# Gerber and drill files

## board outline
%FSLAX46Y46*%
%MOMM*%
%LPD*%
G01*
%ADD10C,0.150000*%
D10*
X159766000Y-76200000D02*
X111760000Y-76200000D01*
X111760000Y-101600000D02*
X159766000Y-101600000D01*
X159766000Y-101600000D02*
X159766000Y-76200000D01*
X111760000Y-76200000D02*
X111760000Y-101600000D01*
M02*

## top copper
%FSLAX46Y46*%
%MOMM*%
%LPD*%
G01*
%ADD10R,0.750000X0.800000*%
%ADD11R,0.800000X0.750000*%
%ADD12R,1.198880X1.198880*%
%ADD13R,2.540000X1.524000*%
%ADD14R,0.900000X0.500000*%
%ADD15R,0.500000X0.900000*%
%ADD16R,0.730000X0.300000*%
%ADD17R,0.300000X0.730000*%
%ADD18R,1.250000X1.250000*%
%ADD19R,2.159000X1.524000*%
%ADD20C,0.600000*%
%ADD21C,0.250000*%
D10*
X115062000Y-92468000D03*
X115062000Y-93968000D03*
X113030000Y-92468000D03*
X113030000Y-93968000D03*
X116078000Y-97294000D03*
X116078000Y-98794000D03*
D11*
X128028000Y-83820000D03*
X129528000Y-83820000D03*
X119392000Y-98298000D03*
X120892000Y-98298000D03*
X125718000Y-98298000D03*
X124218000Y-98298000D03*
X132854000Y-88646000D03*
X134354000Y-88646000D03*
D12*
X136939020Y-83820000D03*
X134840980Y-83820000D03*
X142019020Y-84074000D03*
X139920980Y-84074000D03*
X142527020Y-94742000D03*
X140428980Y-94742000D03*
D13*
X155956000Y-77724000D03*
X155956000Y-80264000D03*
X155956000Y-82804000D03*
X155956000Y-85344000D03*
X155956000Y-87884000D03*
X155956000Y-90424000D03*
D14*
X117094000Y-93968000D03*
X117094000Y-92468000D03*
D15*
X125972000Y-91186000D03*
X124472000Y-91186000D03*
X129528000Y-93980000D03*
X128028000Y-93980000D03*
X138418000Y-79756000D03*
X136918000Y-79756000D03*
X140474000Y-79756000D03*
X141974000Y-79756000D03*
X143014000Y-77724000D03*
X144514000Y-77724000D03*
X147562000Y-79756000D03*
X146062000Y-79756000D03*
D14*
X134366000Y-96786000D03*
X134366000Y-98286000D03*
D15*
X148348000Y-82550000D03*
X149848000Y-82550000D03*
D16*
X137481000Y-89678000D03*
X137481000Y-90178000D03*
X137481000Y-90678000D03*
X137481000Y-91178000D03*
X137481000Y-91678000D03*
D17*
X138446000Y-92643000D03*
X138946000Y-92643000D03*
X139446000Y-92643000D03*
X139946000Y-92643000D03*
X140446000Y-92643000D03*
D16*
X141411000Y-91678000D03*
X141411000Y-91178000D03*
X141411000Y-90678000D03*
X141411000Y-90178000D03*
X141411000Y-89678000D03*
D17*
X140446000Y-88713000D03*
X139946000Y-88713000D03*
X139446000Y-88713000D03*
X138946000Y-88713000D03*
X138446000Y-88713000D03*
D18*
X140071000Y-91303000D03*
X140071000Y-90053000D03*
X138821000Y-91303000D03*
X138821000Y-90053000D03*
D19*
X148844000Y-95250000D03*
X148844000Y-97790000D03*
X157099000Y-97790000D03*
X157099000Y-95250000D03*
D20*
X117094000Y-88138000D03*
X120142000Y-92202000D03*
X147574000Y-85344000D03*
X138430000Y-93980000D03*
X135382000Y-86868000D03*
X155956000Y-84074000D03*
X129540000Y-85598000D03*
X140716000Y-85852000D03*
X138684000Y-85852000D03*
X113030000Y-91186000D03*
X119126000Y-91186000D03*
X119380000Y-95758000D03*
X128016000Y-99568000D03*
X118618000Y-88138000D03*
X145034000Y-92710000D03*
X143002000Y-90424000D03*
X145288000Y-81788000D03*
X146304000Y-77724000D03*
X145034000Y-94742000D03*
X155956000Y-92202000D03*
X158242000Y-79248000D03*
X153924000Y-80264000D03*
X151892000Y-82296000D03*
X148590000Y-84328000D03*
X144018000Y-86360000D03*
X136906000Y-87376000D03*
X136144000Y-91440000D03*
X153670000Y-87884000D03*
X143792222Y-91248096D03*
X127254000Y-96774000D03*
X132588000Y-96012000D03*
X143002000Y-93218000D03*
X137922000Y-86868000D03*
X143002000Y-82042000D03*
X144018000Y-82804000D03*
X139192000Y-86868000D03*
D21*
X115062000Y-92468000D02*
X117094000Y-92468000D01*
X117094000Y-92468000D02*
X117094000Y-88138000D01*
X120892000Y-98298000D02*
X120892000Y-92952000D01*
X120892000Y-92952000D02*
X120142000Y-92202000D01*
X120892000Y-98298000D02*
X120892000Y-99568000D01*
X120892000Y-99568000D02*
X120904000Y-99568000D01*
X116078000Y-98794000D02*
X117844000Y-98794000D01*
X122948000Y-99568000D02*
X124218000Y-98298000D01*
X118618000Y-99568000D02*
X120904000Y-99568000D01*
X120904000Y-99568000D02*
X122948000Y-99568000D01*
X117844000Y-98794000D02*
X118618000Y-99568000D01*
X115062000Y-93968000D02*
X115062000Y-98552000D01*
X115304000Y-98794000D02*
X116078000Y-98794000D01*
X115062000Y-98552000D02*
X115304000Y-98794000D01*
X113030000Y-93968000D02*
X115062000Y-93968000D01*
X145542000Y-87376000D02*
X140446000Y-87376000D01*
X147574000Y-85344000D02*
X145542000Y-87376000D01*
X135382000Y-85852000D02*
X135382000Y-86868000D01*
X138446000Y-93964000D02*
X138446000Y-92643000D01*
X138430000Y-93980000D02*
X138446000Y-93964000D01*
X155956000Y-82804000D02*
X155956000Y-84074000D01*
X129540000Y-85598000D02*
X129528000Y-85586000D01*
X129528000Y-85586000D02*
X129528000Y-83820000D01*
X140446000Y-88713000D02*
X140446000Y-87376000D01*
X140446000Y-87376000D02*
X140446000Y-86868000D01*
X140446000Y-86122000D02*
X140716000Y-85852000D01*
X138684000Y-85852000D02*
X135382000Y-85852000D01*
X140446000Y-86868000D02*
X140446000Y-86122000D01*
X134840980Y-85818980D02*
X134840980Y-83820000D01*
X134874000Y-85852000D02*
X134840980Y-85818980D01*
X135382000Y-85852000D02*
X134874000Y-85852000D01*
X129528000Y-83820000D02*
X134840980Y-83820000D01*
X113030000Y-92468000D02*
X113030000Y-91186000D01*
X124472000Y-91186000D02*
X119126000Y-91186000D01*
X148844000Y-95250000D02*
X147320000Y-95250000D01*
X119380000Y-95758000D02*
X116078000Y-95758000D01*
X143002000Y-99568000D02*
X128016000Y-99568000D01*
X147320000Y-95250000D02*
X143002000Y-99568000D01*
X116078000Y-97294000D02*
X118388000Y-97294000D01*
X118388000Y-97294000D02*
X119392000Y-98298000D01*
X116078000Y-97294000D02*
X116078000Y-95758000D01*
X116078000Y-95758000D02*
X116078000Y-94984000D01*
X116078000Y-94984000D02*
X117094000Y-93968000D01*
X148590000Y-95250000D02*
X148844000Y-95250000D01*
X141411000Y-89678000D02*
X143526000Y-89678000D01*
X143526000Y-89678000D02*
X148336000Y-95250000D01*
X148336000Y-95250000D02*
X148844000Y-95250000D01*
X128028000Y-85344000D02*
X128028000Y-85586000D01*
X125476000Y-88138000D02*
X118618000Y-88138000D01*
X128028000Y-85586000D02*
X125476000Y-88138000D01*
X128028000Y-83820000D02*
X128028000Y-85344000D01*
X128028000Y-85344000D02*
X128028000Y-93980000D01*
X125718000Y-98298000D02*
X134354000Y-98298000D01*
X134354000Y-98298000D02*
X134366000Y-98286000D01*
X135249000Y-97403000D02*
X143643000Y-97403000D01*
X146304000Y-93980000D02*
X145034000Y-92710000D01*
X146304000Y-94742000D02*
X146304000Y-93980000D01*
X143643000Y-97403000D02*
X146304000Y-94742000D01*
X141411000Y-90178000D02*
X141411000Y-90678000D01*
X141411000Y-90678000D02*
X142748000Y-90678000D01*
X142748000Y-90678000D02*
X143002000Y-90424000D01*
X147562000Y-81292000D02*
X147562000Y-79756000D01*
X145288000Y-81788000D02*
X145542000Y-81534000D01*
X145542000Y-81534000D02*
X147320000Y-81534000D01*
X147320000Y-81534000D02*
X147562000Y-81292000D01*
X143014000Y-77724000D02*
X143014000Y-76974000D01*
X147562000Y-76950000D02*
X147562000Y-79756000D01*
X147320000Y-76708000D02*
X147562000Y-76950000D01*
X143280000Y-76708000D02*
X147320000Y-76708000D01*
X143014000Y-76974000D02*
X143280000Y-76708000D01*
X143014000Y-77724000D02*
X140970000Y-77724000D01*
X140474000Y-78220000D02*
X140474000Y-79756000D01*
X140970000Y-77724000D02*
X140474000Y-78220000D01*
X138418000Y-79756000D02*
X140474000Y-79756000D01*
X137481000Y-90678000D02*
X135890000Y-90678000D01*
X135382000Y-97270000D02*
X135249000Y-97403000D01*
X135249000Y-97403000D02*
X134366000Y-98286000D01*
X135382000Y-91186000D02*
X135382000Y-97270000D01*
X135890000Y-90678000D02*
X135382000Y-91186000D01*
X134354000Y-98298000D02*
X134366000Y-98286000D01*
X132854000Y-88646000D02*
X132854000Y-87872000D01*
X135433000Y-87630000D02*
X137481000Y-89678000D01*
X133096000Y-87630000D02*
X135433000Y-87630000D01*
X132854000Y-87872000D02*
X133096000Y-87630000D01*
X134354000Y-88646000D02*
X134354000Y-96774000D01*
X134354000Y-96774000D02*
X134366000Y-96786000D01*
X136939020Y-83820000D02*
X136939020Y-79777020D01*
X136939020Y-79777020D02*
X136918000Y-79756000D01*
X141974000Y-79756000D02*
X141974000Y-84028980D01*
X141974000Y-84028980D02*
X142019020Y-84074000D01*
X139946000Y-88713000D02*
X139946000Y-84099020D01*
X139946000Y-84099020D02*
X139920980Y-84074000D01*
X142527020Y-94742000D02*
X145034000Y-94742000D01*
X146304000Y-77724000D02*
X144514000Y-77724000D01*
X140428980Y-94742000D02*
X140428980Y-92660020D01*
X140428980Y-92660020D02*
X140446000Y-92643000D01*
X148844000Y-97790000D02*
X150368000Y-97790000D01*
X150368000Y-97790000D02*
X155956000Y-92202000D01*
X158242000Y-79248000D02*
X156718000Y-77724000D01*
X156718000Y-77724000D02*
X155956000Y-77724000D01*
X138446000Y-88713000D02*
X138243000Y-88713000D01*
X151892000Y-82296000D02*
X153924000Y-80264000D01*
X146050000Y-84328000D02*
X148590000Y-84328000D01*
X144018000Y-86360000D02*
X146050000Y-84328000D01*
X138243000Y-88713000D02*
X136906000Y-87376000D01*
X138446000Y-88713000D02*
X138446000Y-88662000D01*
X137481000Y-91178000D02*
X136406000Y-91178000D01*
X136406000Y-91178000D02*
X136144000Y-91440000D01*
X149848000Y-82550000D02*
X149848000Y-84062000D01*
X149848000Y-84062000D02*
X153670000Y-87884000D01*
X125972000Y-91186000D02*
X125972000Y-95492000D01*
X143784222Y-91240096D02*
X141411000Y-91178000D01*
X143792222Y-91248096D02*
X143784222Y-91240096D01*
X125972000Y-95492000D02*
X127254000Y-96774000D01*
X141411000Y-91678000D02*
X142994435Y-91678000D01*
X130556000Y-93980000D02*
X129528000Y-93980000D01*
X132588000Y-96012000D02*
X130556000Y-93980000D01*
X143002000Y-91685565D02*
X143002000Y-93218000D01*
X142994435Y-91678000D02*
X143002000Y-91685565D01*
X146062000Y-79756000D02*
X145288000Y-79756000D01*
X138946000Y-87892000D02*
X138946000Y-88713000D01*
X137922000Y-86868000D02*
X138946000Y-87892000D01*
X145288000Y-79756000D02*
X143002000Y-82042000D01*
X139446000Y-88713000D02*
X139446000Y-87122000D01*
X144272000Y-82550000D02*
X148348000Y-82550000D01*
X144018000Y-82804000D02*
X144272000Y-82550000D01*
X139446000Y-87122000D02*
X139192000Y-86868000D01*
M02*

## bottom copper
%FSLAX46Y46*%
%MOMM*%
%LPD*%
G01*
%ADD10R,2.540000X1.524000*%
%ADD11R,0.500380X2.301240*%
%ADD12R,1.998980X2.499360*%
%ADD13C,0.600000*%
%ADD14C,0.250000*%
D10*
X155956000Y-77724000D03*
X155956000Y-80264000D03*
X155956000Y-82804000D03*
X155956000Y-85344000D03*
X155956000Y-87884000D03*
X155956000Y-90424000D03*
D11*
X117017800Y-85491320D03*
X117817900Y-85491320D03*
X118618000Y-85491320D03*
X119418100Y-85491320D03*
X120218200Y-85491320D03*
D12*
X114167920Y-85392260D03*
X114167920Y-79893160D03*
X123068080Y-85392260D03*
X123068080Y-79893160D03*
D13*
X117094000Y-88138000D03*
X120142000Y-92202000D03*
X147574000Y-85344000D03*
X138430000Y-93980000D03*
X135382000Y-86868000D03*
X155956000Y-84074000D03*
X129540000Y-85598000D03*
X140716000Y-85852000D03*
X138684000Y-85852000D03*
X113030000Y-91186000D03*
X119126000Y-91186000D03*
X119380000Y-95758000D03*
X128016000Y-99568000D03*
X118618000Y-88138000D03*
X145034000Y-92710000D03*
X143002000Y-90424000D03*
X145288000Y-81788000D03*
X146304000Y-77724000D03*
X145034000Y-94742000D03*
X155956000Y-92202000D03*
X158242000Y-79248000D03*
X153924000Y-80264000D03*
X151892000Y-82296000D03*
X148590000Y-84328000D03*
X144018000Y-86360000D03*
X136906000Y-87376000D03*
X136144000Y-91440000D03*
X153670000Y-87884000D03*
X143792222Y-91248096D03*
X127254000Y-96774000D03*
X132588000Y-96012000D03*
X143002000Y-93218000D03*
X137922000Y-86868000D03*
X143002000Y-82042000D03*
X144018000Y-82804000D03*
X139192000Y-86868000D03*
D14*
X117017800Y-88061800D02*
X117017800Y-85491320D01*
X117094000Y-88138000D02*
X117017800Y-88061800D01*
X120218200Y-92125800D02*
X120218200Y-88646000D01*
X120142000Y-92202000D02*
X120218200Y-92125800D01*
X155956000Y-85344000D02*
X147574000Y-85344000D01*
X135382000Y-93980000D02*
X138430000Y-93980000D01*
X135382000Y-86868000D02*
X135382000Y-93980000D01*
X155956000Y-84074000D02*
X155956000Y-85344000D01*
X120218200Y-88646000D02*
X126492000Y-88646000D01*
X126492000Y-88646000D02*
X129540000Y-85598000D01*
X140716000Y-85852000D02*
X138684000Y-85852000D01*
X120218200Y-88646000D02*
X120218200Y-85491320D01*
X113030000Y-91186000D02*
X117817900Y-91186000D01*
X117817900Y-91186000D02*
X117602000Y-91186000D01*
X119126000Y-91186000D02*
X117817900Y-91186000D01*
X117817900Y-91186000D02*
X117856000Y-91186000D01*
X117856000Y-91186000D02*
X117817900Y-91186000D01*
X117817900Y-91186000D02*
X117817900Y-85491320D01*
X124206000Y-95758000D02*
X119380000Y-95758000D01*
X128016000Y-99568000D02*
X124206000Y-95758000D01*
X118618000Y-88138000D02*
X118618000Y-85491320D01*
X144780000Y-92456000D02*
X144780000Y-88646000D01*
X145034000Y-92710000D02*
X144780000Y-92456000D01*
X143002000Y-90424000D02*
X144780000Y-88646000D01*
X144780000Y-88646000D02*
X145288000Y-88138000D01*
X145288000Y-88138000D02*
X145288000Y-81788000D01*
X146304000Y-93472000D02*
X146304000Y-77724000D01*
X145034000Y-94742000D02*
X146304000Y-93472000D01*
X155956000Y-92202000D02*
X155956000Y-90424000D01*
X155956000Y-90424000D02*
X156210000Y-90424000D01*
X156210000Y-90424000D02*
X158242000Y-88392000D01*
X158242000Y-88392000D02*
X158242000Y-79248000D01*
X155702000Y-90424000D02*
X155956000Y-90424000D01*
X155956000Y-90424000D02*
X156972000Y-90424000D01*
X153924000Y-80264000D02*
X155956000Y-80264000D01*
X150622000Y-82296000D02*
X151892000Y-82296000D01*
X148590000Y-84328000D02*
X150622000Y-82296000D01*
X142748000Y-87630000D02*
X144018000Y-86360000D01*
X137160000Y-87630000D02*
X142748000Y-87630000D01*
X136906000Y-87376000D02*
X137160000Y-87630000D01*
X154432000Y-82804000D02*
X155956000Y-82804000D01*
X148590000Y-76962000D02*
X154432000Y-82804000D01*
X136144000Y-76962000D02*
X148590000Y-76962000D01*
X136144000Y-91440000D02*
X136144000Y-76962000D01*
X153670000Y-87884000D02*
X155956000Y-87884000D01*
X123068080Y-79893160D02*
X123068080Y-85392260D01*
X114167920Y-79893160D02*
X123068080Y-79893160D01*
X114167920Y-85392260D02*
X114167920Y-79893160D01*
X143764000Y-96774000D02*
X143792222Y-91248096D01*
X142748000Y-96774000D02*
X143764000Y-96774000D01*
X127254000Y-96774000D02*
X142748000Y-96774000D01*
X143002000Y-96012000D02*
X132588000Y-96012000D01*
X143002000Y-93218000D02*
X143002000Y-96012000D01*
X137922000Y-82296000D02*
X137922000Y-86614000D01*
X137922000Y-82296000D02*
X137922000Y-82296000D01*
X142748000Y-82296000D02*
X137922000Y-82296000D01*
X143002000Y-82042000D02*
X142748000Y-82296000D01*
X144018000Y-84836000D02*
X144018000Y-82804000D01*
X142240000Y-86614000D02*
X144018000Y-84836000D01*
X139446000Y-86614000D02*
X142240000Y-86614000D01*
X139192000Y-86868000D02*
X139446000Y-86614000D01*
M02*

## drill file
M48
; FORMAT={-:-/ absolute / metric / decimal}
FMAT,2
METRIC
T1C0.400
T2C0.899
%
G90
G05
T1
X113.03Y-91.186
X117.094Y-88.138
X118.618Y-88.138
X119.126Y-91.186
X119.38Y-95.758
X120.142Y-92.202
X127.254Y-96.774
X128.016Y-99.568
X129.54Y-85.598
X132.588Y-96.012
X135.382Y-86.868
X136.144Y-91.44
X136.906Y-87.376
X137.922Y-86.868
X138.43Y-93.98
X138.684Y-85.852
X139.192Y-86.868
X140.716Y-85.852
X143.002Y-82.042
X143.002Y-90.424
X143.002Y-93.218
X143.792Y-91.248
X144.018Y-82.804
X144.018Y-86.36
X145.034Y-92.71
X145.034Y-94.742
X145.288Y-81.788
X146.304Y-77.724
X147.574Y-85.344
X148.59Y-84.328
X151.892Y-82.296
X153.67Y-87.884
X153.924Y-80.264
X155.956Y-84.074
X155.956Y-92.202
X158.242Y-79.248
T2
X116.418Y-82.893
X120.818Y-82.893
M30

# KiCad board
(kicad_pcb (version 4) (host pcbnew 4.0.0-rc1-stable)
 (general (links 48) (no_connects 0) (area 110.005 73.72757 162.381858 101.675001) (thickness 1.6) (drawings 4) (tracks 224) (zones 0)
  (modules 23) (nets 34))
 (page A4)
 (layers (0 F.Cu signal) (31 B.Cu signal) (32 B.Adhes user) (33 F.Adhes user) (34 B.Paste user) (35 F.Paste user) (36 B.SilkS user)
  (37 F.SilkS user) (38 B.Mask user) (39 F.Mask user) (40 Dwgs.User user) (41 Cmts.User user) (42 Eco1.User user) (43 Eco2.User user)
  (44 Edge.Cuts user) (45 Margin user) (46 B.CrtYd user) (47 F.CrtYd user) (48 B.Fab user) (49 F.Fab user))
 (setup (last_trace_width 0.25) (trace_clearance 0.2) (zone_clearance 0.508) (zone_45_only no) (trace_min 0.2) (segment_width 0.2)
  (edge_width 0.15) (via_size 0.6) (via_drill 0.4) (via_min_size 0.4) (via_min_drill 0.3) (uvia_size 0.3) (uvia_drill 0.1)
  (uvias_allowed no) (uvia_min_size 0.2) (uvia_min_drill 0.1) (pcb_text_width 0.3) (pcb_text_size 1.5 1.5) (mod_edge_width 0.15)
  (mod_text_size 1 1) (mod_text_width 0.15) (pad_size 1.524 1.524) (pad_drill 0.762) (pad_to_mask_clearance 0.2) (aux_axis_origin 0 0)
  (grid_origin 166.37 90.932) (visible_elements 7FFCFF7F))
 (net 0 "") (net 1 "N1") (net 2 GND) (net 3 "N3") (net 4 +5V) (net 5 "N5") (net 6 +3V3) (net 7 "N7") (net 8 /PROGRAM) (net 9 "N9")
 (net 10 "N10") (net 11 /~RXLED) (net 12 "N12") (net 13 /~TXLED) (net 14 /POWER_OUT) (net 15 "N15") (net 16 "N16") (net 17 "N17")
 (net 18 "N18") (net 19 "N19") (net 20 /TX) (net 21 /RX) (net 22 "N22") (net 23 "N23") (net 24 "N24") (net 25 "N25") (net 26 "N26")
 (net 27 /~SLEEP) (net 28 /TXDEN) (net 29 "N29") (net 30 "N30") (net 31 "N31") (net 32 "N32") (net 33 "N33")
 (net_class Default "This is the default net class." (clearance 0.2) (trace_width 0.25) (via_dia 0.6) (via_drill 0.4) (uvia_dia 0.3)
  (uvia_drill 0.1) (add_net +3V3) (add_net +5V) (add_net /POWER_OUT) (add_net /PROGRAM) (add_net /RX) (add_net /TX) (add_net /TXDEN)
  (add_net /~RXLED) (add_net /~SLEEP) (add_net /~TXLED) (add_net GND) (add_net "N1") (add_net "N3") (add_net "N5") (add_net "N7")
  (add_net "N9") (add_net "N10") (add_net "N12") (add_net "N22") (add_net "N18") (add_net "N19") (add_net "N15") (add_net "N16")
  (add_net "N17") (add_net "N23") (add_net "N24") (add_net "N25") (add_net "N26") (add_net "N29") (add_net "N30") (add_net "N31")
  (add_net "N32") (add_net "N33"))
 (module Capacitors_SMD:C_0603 (layer F.Cu) (at 115.062 93.218 270)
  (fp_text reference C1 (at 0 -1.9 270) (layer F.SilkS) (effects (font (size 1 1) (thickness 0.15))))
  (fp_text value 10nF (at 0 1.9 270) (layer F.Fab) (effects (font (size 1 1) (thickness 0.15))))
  (pad 1 smd rect (at -0.75 0 270) (size 0.8 0.75) (layers F.Cu F.Paste F.Mask) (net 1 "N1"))
  (pad 2 smd rect (at 0.75 0 270) (size 0.8 0.75) (layers F.Cu F.Paste F.Mask) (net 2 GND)))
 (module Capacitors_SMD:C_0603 (layer F.Cu) (at 113.03 93.218 270)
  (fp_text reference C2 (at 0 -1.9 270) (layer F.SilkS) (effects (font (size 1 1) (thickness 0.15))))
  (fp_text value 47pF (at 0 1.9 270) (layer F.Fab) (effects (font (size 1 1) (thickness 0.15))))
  (pad 1 smd rect (at -0.75 0 270) (size 0.8 0.75) (layers F.Cu F.Paste F.Mask) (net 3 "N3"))
  (pad 2 smd rect (at 0.75 0 270) (size 0.8 0.75) (layers F.Cu F.Paste F.Mask) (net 2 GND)))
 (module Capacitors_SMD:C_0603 (layer F.Cu) (at 116.078 98.044 270)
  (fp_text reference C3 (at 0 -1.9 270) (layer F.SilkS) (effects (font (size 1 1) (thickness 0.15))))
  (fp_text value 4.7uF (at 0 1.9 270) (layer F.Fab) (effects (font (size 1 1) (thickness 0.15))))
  (pad 1 smd rect (at -0.75 0 270) (size 0.8 0.75) (layers F.Cu F.Paste F.Mask) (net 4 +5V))
  (pad 2 smd rect (at 0.75 0 270) (size 0.8 0.75) (layers F.Cu F.Paste F.Mask) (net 2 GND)))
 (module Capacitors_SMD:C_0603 (layer F.Cu) (at 128.778 83.82)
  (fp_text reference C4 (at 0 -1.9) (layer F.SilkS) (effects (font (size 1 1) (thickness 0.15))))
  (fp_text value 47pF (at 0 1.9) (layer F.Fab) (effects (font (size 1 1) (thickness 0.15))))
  (pad 1 smd rect (at -0.75 0) (size 0.8 0.75) (layers F.Cu F.Paste F.Mask) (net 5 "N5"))
  (pad 2 smd rect (at 0.75 0) (size 0.8 0.75) (layers F.Cu F.Paste F.Mask) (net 2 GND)))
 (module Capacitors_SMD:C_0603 (layer F.Cu) (at 120.142 98.298)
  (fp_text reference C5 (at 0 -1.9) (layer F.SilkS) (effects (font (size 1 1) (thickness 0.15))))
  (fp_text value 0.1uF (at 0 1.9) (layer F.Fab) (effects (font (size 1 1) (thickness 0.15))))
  (pad 1 smd rect (at -0.75 0) (size 0.8 0.75) (layers F.Cu F.Paste F.Mask) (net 4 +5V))
  (pad 2 smd rect (at 0.75 0) (size 0.8 0.75) (layers F.Cu F.Paste F.Mask) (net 2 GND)))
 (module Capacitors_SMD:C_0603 (layer F.Cu) (at 124.968 98.298 180)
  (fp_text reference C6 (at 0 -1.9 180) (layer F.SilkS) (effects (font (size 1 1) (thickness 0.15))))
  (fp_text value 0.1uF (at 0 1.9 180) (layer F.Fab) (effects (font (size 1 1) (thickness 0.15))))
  (pad 1 smd rect (at -0.75 0 180) (size 0.8 0.75) (layers F.Cu F.Paste F.Mask) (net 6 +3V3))
  (pad 2 smd rect (at 0.75 0 180) (size 0.8 0.75) (layers F.Cu F.Paste F.Mask) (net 2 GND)))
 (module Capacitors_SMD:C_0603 (layer F.Cu) (at 133.604 88.646)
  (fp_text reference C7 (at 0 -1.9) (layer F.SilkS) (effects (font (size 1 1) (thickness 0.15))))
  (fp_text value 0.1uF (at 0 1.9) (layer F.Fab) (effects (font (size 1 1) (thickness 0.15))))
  (pad 1 smd rect (at -0.75 0) (size 0.8 0.75) (layers F.Cu F.Paste F.Mask) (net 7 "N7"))
  (pad 2 smd rect (at 0.75 0) (size 0.8 0.75) (layers F.Cu F.Paste F.Mask) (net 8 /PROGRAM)))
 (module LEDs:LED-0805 (layer F.Cu) (at 135.89 83.82)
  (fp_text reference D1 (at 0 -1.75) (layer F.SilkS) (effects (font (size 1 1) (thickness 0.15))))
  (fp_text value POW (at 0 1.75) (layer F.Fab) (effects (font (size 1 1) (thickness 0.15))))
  (pad 2 smd rect (at 1.04902 0 180) (size 1.19888 1.19888) (layers F.Cu F.Paste F.Mask) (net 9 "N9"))
  (pad 1 smd rect (at -1.04902 0 180) (size 1.19888 1.19888) (layers F.Cu F.Paste F.Mask) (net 2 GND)))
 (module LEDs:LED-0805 (layer F.Cu) (at 140.97 84.074)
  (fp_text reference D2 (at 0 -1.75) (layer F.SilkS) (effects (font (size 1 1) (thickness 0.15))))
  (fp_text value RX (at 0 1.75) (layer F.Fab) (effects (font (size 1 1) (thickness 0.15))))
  (pad 2 smd rect (at 1.04902 0 180) (size 1.19888 1.19888) (layers F.Cu F.Paste F.Mask) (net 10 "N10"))
  (pad 1 smd rect (at -1.04902 0 180) (size 1.19888 1.19888) (layers F.Cu F.Paste F.Mask) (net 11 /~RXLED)))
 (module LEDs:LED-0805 (layer F.Cu) (at 141.478 94.742)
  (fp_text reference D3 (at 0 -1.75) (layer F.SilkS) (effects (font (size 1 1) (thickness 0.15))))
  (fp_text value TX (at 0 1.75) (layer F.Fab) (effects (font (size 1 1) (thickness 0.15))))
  (pad 2 smd rect (at 1.04902 0 180) (size 1.19888 1.19888) (layers F.Cu F.Paste F.Mask) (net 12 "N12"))
  (pad 1 smd rect (at -1.04902 0 180) (size 1.19888 1.19888) (layers F.Cu F.Paste F.Mask) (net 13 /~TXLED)))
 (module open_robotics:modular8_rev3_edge (layer F.Cu) (at 155.956 82.804 270)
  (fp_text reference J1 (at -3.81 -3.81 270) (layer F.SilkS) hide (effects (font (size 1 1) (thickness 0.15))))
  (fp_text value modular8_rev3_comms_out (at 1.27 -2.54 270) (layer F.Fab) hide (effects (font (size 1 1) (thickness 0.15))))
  (pad 1 smd rect (at -5.08 0 270) (size 1.524 2.54) (layers F.Cu F.Paste F.Mask) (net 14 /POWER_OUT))
  (pad 3 smd rect (at -2.54 0 270) (size 1.524 2.54) (layers F.Cu F.Paste F.Mask) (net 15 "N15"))
  (pad 5 smd rect (at 0 0 270) (size 1.524 2.54) (layers F.Cu F.Paste F.Mask) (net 2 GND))
  (pad 7 smd rect (at 2.54 0 270) (size 1.524 2.54) (layers F.Cu F.Paste F.Mask) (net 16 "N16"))
  (pad 9 smd rect (at 5.08 0 270) (size 1.524 2.54) (layers F.Cu F.Paste F.Mask) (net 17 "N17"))
  (pad 11 smd rect (at 7.62 0 270) (size 1.524 2.54) (layers F.Cu F.Paste F.Mask) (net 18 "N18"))
  (pad 2 smd rect (at -5.08 0 270) (size 1.524 2.54) (layers B.Cu F.Paste F.Mask) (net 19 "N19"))
  (pad 4 smd rect (at -2.54 0 270) (size 1.524 2.54) (layers B.Cu F.Paste F.Mask) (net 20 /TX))
  (pad 6 smd rect (at 0 0 270) (size 1.524 2.54) (layers B.Cu F.Paste F.Mask) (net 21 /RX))
  (pad 8 smd rect (at 2.54 0 270) (size 1.524 2.54) (layers B.Cu F.Paste F.Mask) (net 2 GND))
  (pad 10 smd rect (at 5.08 0 270) (size 1.524 2.54) (layers B.Cu F.Paste F.Mask) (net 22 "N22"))
  (pad 12 smd rect (at 7.62 0 270) (size 1.524 2.54) (layers B.Cu F.Paste F.Mask) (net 14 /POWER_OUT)))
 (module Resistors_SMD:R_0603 (layer F.Cu) (at 117.094 93.218 90)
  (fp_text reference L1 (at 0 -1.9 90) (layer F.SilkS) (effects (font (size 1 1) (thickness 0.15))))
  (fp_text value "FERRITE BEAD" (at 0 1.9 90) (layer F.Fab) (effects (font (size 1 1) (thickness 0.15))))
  (pad 1 smd rect (at -0.75 0 90) (size 0.5 0.9) (layers F.Cu F.Paste F.Mask) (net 4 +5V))
  (pad 2 smd rect (at 0.75 0 90) (size 0.5 0.9) (layers F.Cu F.Paste F.Mask) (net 1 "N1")))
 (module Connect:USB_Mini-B (layer B.Cu) (at 118.618 82.042 270)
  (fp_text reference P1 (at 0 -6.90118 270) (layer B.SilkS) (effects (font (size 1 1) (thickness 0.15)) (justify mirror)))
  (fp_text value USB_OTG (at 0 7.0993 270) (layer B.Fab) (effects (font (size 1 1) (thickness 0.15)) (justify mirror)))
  (pad 1 smd rect (at 3.44932 1.6002 270) (size 2.30124 0.50038) (layers B.Cu B.Paste B.Mask) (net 1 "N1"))
  (pad 2 smd rect (at 3.44932 0.8001 270) (size 2.30124 0.50038) (layers B.Cu B.Paste B.Mask) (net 3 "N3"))
  (pad 3 smd rect (at 3.44932 0 270) (size 2.30124 0.50038) (layers B.Cu B.Paste B.Mask) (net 5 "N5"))
  (pad 4 smd rect (at 3.44932 -0.8001 270) (size 2.30124 0.50038) (layers B.Cu B.Paste B.Mask) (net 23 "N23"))
  (pad 5 smd rect (at 3.44932 -1.6002 270) (size 2.30124 0.50038) (layers B.Cu B.Paste B.Mask) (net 2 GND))
  (pad 6 smd rect (at 3.35026 4.45008 270) (size 2.49936 1.99898) (layers B.Cu B.Paste B.Mask) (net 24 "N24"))
  (pad 6 smd rect (at -2.14884 4.45008 270) (size 2.49936 1.99898) (layers B.Cu B.Paste B.Mask) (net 24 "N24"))
  (pad 6 smd rect (at 3.35026 -4.45008 270) (size 2.49936 1.99898) (layers B.Cu B.Paste B.Mask) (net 24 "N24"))
  (pad 6 smd rect (at -2.14884 -4.45008 270) (size 2.49936 1.99898) (layers B.Cu B.Paste B.Mask) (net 24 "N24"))
  (pad "" np_thru_hole circle (at 0.8509 2.19964 270) (size 0.89916 0.89916) (drill 0.89916) (layers *.Cu *.Mask B.SilkS))
  (pad "" np_thru_hole circle (at 0.8509 -2.19964 270) (size 0.89916 0.89916) (drill 0.89916) (layers *.Cu *.Mask B.SilkS)))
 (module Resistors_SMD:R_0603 (layer F.Cu) (at 125.222 91.186 180)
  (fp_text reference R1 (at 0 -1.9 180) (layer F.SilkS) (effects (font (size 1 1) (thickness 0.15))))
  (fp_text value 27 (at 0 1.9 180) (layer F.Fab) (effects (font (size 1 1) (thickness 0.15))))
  (pad 1 smd rect (at -0.75 0 180) (size 0.5 0.9) (layers F.Cu F.Paste F.Mask) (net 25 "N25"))
  (pad 2 smd rect (at 0.75 0 180) (size 0.5 0.9) (layers F.Cu F.Paste F.Mask) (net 3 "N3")))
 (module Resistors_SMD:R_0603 (layer F.Cu) (at 128.778 93.98 180)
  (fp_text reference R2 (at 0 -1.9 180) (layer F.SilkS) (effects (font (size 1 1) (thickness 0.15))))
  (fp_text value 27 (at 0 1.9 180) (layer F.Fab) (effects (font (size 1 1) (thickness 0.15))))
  (pad 1 smd rect (at -0.75 0 180) (size 0.5 0.9) (layers F.Cu F.Paste F.Mask) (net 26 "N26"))
  (pad 2 smd rect (at 0.75 0 180) (size 0.5 0.9) (layers F.Cu F.Paste F.Mask) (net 5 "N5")))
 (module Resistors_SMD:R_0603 (layer F.Cu) (at 137.668 79.756 180)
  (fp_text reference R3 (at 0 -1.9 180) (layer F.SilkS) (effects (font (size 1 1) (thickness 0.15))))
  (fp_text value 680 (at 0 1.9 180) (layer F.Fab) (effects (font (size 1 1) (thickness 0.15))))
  (pad 1 smd rect (at -0.75 0 180) (size 0.5 0.9) (layers F.Cu F.Paste F.Mask) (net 6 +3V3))
  (pad 2 smd rect (at 0.75 0 180) (size 0.5 0.9) (layers F.Cu F.Paste F.Mask) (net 9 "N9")))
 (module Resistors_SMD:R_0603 (layer F.Cu) (at 141.224 79.756)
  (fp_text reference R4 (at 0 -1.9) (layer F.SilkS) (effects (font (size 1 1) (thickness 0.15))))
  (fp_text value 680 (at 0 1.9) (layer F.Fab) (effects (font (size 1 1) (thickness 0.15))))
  (pad 1 smd rect (at -0.75 0) (size 0.5 0.9) (layers F.Cu F.Paste F.Mask) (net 6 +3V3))
  (pad 2 smd rect (at 0.75 0) (size 0.5 0.9) (layers F.Cu F.Paste F.Mask) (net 10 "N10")))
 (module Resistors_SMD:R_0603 (layer F.Cu) (at 143.764 77.724)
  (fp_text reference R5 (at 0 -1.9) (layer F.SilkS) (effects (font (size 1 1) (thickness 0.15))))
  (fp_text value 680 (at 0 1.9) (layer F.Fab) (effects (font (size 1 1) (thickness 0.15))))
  (pad 1 smd rect (at -0.75 0) (size 0.5 0.9) (layers F.Cu F.Paste F.Mask) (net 6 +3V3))
  (pad 2 smd rect (at 0.75 0) (size 0.5 0.9) (layers F.Cu F.Paste F.Mask) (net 12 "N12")))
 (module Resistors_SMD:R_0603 (layer F.Cu) (at 146.812 79.756 180)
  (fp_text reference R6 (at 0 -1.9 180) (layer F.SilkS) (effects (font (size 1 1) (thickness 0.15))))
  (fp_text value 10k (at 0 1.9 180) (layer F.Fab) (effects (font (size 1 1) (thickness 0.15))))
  (pad 1 smd rect (at -0.75 0 180) (size 0.5 0.9) (layers F.Cu F.Paste F.Mask) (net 6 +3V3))
  (pad 2 smd rect (at 0.75 0 180) (size 0.5 0.9) (layers F.Cu F.Paste F.Mask) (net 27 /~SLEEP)))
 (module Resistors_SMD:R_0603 (layer F.Cu) (at 134.366 97.536 270)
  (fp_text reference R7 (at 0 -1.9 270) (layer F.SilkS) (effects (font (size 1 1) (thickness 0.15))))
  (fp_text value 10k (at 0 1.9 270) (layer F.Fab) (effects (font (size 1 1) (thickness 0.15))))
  (pad 1 smd rect (at -0.75 0 270) (size 0.5 0.9) (layers F.Cu F.Paste F.Mask) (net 8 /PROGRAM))
  (pad 2 smd rect (at 0.75 0 270) (size 0.5 0.9) (layers F.Cu F.Paste F.Mask) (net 6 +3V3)))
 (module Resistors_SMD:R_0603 (layer F.Cu) (at 149.098 82.55)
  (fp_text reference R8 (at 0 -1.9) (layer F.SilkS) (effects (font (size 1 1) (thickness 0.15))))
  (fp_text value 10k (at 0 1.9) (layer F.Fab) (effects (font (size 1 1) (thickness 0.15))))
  (pad 1 smd rect (at -0.75 0) (size 0.5 0.9) (layers F.Cu F.Paste F.Mask) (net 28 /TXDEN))
  (pad 2 smd rect (at 0.75 0) (size 0.5 0.9) (layers F.Cu F.Paste F.Mask) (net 22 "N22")))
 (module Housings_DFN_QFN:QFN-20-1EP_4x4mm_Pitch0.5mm (layer F.Cu) (at 139.446 90.678)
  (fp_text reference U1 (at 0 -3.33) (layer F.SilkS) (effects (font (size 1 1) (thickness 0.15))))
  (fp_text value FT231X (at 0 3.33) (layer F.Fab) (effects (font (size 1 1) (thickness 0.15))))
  (pad 1 smd rect (at -1.965 -1) (size 0.73 0.3) (layers F.Cu F.Paste F.Mask) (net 7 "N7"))
  (pad 2 smd rect (at -1.965 -0.5) (size 0.73 0.3) (layers F.Cu F.Paste F.Mask) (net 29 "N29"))
  (pad 3 smd rect (at -1.965 0) (size 0.73 0.3) (layers F.Cu F.Paste F.Mask) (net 6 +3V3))
  (pad 4 smd rect (at -1.965 0.5) (size 0.73 0.3) (layers F.Cu F.Paste F.Mask) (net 21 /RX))
  (pad 5 smd rect (at -1.965 1) (size 0.73 0.3) (layers F.Cu F.Paste F.Mask) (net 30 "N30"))
  (pad 6 smd rect (at -1 1.965 90) (size 0.73 0.3) (layers F.Cu F.Paste F.Mask) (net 2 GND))
  (pad 7 smd rect (at -0.5 1.965 90) (size 0.73 0.3) (layers F.Cu F.Paste F.Mask) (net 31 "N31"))
  (pad 8 smd rect (at 0 1.965 90) (size 0.73 0.3) (layers F.Cu F.Paste F.Mask) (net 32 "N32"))
  (pad 9 smd rect (at 0.5 1.965 90) (size 0.73 0.3) (layers F.Cu F.Paste F.Mask) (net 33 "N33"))
  (pad 10 smd rect (at 1 1.965 90) (size 0.73 0.3) (layers F.Cu F.Paste F.Mask) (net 13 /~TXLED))
  (pad 11 smd rect (at 1.965 1) (size 0.73 0.3) (layers F.Cu F.Paste F.Mask) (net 26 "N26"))
  (pad 12 smd rect (at 1.965 0.5) (size 0.73 0.3) (layers F.Cu F.Paste F.Mask) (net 25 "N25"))
  (pad 13 smd rect (at 1.965 0) (size 0.73 0.3) (layers F.Cu F.Paste F.Mask) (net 6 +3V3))
  (pad 14 smd rect (at 1.965 -0.5) (size 0.73 0.3) (layers F.Cu F.Paste F.Mask) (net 6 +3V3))
  (pad 15 smd rect (at 1.965 -1) (size 0.73 0.3) (layers F.Cu F.Paste F.Mask) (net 4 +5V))
  (pad 16 smd rect (at 1 -1.965 90) (size 0.73 0.3) (layers F.Cu F.Paste F.Mask) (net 2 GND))
  (pad 17 smd rect (at 0.5 -1.965 90) (size 0.73 0.3) (layers F.Cu F.Paste F.Mask) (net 11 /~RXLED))
  (pad 18 smd rect (at 0 -1.965 90) (size 0.73 0.3) (layers F.Cu F.Paste F.Mask) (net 28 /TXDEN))
  (pad 19 smd rect (at -0.5 -1.965 90) (size 0.73 0.3) (layers F.Cu F.Paste F.Mask) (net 27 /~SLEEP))
  (pad 20 smd rect (at -1 -1.965 90) (size 0.73 0.3) (layers F.Cu F.Paste F.Mask) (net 20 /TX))
  (pad 21 smd rect (at 0.625 0.625) (size 1.25 1.25) (layers F.Cu F.Paste F.Mask) (solder_paste_margin_ratio -0.2))
  (pad 21 smd rect (at 0.625 -0.625) (size 1.25 1.25) (layers F.Cu F.Paste F.Mask) (solder_paste_margin_ratio -0.2))
  (pad 21 smd rect (at -0.625 0.625) (size 1.25 1.25) (layers F.Cu F.Paste F.Mask) (solder_paste_margin_ratio -0.2))
  (pad 21 smd rect (at -0.625 -0.625) (size 1.25 1.25) (layers F.Cu F.Paste F.Mask) (solder_paste_margin_ratio -0.2)))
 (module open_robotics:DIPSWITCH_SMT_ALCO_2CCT (layer F.Cu) (at 148.844 95.25)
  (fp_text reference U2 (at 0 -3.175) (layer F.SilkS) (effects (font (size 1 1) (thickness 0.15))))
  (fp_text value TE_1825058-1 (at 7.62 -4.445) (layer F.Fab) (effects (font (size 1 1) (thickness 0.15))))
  (pad 1 smd rect (at 0 0) (size 2.159 1.524) (layers F.Cu F.Paste F.Mask) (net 4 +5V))
  (pad 2 smd rect (at 0 2.54) (size 2.159 1.524) (layers F.Cu F.Paste F.Mask) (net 14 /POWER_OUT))
  (pad 3 smd rect (at 8.255 2.54) (size 2.159 1.524) (layers F.Cu F.Paste F.Mask))
  (pad 4 smd rect (at 8.255 0) (size 2.159 1.524) (layers F.Cu F.Paste F.Mask)))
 (gr_line (start 159.766 76.2) (end 111.76 76.2) (angle 90) (layer Edge.Cuts) (width 0.15))
 (gr_line (start 111.76 101.6) (end 159.766 101.6) (angle 90) (layer Edge.Cuts) (width 0.15))
 (gr_line (start 159.766 101.6) (end 159.766 76.2) (angle 90) (layer Edge.Cuts) (width 0.15))
 (gr_line (start 111.76 76.2) (end 111.76 101.6) (angle 90) (layer Edge.Cuts) (width 0.15))
 (segment (start 115.062 92.468) (end 117.094 92.468) (width 0.25) (layer F.Cu) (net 1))
 (segment (start 117.094 92.468) (end 117.094 88.138) (width 0.25) (layer F.Cu) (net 1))
 (segment (start 117.0178 88.0618) (end 117.0178 85.49132) (width 0.25) (layer B.Cu) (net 1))
 (segment (start 117.094 88.138) (end 117.0178 88.0618) (width 0.25) (layer B.Cu) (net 1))
 (via (at 117.094 88.138) (size 0.6) (drill 0.4) (layers F.Cu B.Cu) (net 1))
 (segment (start 120.892 98.298) (end 120.892 92.952) (width 0.25) (layer F.Cu) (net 2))
 (segment (start 120.2182 92.1258) (end 120.2182 88.646) (width 0.25) (layer B.Cu) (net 2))
 (segment (start 120.142 92.202) (end 120.2182 92.1258) (width 0.25) (layer B.Cu) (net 2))
 (via (at 120.142 92.202) (size 0.6) (drill 0.4) (layers F.Cu B.Cu) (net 2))
 (segment (start 120.892 92.952) (end 120.142 92.202) (width 0.25) (layer F.Cu) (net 2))
 (segment (start 120.892 98.298) (end 120.892 99.568) (width 0.25) (layer F.Cu) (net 2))
 (segment (start 120.892 99.568) (end 120.904 99.568) (width 0.25) (layer F.Cu) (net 2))
 (segment (start 116.078 98.794) (end 117.844 98.794) (width 0.25) (layer F.Cu) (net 2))
 (segment (start 122.948 99.568) (end 124.218 98.298) (width 0.25) (layer F.Cu) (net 2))
 (segment (start 118.618 99.568) (end 120.904 99.568) (width 0.25) (layer F.Cu) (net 2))
 (segment (start 120.904 99.568) (end 122.948 99.568) (width 0.25) (layer F.Cu) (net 2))
 (segment (start 117.844 98.794) (end 118.618 99.568) (width 0.25) (layer F.Cu) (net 2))
 (segment (start 115.062 93.968) (end 115.062 98.552) (width 0.25) (layer F.Cu) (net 2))
 (segment (start 115.304 98.794) (end 116.078 98.794) (width 0.25) (layer F.Cu) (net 2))
 (segment (start 115.062 98.552) (end 115.304 98.794) (width 0.25) (layer F.Cu) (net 2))
 (segment (start 113.03 93.968) (end 115.062 93.968) (width 0.25) (layer F.Cu) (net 2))
 (segment (start 155.956 85.344) (end 147.574 85.344) (width 0.25) (layer B.Cu) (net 2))
 (segment (start 145.542 87.376) (end 140.446 87.376) (width 0.25) (layer F.Cu) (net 2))
 (segment (start 147.574 85.344) (end 145.542 87.376) (width 0.25) (layer F.Cu) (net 2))
 (via (at 147.574 85.344) (size 0.6) (drill 0.4) (layers F.Cu B.Cu) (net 2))
 (segment (start 135.382 85.852) (end 135.382 86.868) (width 0.25) (layer F.Cu) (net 2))
 (segment (start 138.446 93.964) (end 138.446 92.643) (width 0.25) (layer F.Cu) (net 2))
 (segment (start 138.43 93.98) (end 138.446 93.964) (width 0.25) (layer F.Cu) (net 2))
 (via (at 138.43 93.98) (size 0.6) (drill 0.4) (layers F.Cu B.Cu) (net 2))
 (segment (start 135.382 93.98) (end 138.43 93.98) (width 0.25) (layer B.Cu) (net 2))
 (segment (start 135.382 86.868) (end 135.382 93.98) (width 0.25) (layer B.Cu) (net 2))
 (via (at 135.382 86.868) (size 0.6) (drill 0.4) (layers F.Cu B.Cu) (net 2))
 (segment (start 155.956 82.804) (end 155.956 84.074) (width 0.25) (layer F.Cu) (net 2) (status 10))
 (segment (start 155.956 84.074) (end 155.956 85.344) (width 0.25) (layer B.Cu) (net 2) (status 20))
 (via (at 155.956 84.074) (size 0.6) (drill 0.4) (layers F.Cu B.Cu) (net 2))
 (segment (start 120.2182 88.646) (end 126.492 88.646) (width 0.25) (layer B.Cu) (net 2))
 (segment (start 126.492 88.646) (end 129.54 85.598) (width 0.25) (layer B.Cu) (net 2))
 (via (at 129.54 85.598) (size 0.6) (drill 0.4) (layers F.Cu B.Cu) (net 2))
 (segment (start 129.54 85.598) (end 129.528 85.586) (width 0.25) (layer F.Cu) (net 2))
 (segment (start 129.528 85.586) (end 129.528 83.82) (width 0.25) (layer F.Cu) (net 2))
 (segment (start 140.446 88.713) (end 140.446 87.376) (width 0.25) (layer F.Cu) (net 2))
 (segment (start 140.446 87.376) (end 140.446 86.868) (width 0.25) (layer F.Cu) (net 2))
 (segment (start 140.446 86.122) (end 140.716 85.852) (width 0.25) (layer F.Cu) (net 2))
 (via (at 140.716 85.852) (size 0.6) (drill 0.4) (layers F.Cu B.Cu) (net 2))
 (segment (start 140.716 85.852) (end 138.684 85.852) (width 0.25) (layer B.Cu) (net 2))
 (via (at 138.684 85.852) (size 0.6) (drill 0.4) (layers F.Cu B.Cu) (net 2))
 (segment (start 138.684 85.852) (end 135.382 85.852) (width 0.25) (layer F.Cu) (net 2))
 (segment (start 140.446 86.868) (end 140.446 86.122) (width 0.25) (layer F.Cu) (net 2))
 (segment (start 134.84098 85.81898) (end 134.84098 83.82) (width 0.25) (layer F.Cu) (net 2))
 (segment (start 134.874 85.852) (end 134.84098 85.81898) (width 0.25) (layer F.Cu) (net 2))
 (segment (start 135.382 85.852) (end 134.874 85.852) (width 0.25) (layer F.Cu) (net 2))
 (segment (start 120.2182 88.646) (end 120.2182 85.49132) (width 0.25) (layer B.Cu) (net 2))
 (segment (start 129.528 83.82) (end 134.84098 83.82) (width 0.25) (layer F.Cu) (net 2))
 (segment (start 113.03 92.468) (end 113.03 91.186) (width 0.25) (layer F.Cu) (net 3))
 (segment (start 113.03 91.186) (end 117.8179 91.186) (width 0.25) (layer B.Cu) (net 3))
 (via (at 113.03 91.186) (size 0.6) (drill 0.4) (layers F.Cu B.Cu) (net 3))
 (segment (start 117.8179 91.186) (end 117.602 91.186) (width 0.25) (layer B.Cu) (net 3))
 (segment (start 124.472 91.186) (end 119.126 91.186) (width 0.25) (layer F.Cu) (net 3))
 (segment (start 119.126 91.186) (end 117.8179 91.186) (width 0.25) (layer B.Cu) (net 3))
 (via (at 119.126 91.186) (size 0.6) (drill 0.4) (layers F.Cu B.Cu) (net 3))
 (segment (start 117.8179 91.186) (end 117.856 91.186) (width 0.25) (layer B.Cu) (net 3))
 (segment (start 117.856 91.186) (end 117.8179 91.186) (width 0.25) (layer B.Cu) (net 3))
 (segment (start 117.8179 91.186) (end 117.8179 85.49132) (width 0.25) (layer B.Cu) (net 3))
 (segment (start 148.844 95.25) (end 147.32 95.25) (width 0.25) (layer F.Cu) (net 4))
 (segment (start 119.38 95.758) (end 116.078 95.758) (width 0.25) (layer F.Cu) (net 4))
 (via (at 119.38 95.758) (size 0.6) (drill 0.4) (layers F.Cu B.Cu) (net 4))
 (segment (start 124.206 95.758) (end 119.38 95.758) (width 0.25) (layer B.Cu) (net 4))
 (segment (start 128.016 99.568) (end 124.206 95.758) (width 0.25) (layer B.Cu) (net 4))
 (via (at 128.016 99.568) (size 0.6) (drill 0.4) (layers F.Cu B.Cu) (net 4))
 (segment (start 143.002 99.568) (end 128.016 99.568) (width 0.25) (layer F.Cu) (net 4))
 (segment (start 147.32 95.25) (end 143.002 99.568) (width 0.25) (layer F.Cu) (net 4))
 (segment (start 116.078 97.294) (end 118.388 97.294) (width 0.25) (layer F.Cu) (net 4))
 (segment (start 118.388 97.294) (end 119.392 98.298) (width 0.25) (layer F.Cu) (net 4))
 (segment (start 116.078 97.294) (end 116.078 95.758) (width 0.25) (layer F.Cu) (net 4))
 (segment (start 116.078 95.758) (end 116.078 94.984) (width 0.25) (layer F.Cu) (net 4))
 (segment (start 116.078 94.984) (end 117.094 93.968) (width 0.25) (layer F.Cu) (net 4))
 (segment (start 148.59 95.25) (end 148.844 95.25) (width 0.25) (layer F.Cu) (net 4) (status 30))
 (segment (start 141.411 89.678) (end 143.526 89.678) (width 0.25) (layer F.Cu) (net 4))
 (segment (start 143.526 89.678) (end 148.336 95.25) (width 0.25) (layer F.Cu) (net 4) (status 20))
 (segment (start 148.336 95.25) (end 148.844 95.25) (width 0.25) (layer F.Cu) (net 4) (status 30))
 (segment (start 128.028 85.344) (end 128.028 85.586) (width 0.25) (layer F.Cu) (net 5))
 (segment (start 118.618 88.138) (end 118.618 85.49132) (width 0.25) (layer B.Cu) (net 5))
 (via (at 118.618 88.138) (size 0.6) (drill 0.4) (layers F.Cu B.Cu) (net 5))
 (segment (start 125.476 88.138) (end 118.618 88.138) (width 0.25) (layer F.Cu) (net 5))
 (segment (start 128.028 85.586) (end 125.476 88.138) (width 0.25) (layer F.Cu) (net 5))
 (segment (start 128.028 83.82) (end 128.028 85.344) (width 0.25) (layer F.Cu) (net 5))
 (segment (start 128.028 85.344) (end 128.028 93.98) (width 0.25) (layer F.Cu) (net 5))
 (segment (start 125.718 98.298) (end 134.354 98.298) (width 0.25) (layer F.Cu) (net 6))
 (segment (start 134.354 98.298) (end 134.366 98.286) (width 0.25) (layer F.Cu) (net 6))
 (segment (start 135.249 97.403) (end 143.643 97.403) (width 0.25) (layer F.Cu) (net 6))
 (segment (start 144.78 92.456) (end 144.78 88.646) (width 0.25) (layer B.Cu) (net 6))
 (segment (start 145.034 92.71) (end 144.78 92.456) (width 0.25) (layer B.Cu) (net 6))
 (via (at 145.034 92.71) (size 0.6) (drill 0.4) (layers F.Cu B.Cu) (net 6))
 (segment (start 146.304 93.98) (end 145.034 92.71) (width 0.25) (layer F.Cu) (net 6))
 (segment (start 146.304 94.742) (end 146.304 93.98) (width 0.25) (layer F.Cu) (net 6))
 (segment (start 143.643 97.403) (end 146.304 94.742) (width 0.25) (layer F.Cu) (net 6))
 (segment (start 141.411 90.178) (end 141.411 90.678) (width 0.25) (layer F.Cu) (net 6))
 (segment (start 141.411 90.678) (end 142.748 90.678) (width 0.25) (layer F.Cu) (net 6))
 (segment (start 142.748 90.678) (end 143.002 90.424) (width 0.25) (layer F.Cu) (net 6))
 (via (at 143.002 90.424) (size 0.6) (drill 0.4) (layers F.Cu B.Cu) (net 6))
 (segment (start 143.002 90.424) (end 144.78 88.646) (width 0.25) (layer B.Cu) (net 6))
 (segment (start 147.562 81.292) (end 147.562 79.756) (width 0.25) (layer F.Cu) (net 6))
 (segment (start 144.78 88.646) (end 145.288 88.138) (width 0.25) (layer B.Cu) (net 6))
 (segment (start 145.288 88.138) (end 145.288 81.788) (width 0.25) (layer B.Cu) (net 6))
 (via (at 145.288 81.788) (size 0.6) (drill 0.4) (layers F.Cu B.Cu) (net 6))
 (segment (start 145.288 81.788) (end 145.542 81.534) (width 0.25) (layer F.Cu) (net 6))
 (segment (start 145.542 81.534) (end 147.32 81.534) (width 0.25) (layer F.Cu) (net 6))
 (segment (start 147.32 81.534) (end 147.562 81.292) (width 0.25) (layer F.Cu) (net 6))
 (segment (start 143.014 77.724) (end 143.014 76.974) (width 0.25) (layer F.Cu) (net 6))
 (segment (start 147.562 76.95) (end 147.562 79.756) (width 0.25) (layer F.Cu) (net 6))
 (segment (start 147.32 76.708) (end 147.562 76.95) (width 0.25) (layer F.Cu) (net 6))
 (segment (start 143.28 76.708) (end 147.32 76.708) (width 0.25) (layer F.Cu) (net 6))
 (segment (start 143.014 76.974) (end 143.28 76.708) (width 0.25) (layer F.Cu) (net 6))
 (segment (start 143.014 77.724) (end 140.97 77.724) (width 0.25) (layer F.Cu) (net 6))
 (segment (start 140.474 78.22) (end 140.474 79.756) (width 0.25) (layer F.Cu) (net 6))
 (segment (start 140.97 77.724) (end 140.474 78.22) (width 0.25) (layer F.Cu) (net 6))
 (segment (start 138.418 79.756) (end 140.474 79.756) (width 0.25) (layer F.Cu) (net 6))
 (segment (start 137.481 90.678) (end 135.89 90.678) (width 0.25) (layer F.Cu) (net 6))
 (segment (start 135.382 97.27) (end 135.249 97.403) (width 0.25) (layer F.Cu) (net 6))
 (segment (start 135.249 97.403) (end 134.366 98.286) (width 0.25) (layer F.Cu) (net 6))
 (segment (start 135.382 91.186) (end 135.382 97.27) (width 0.25) (layer F.Cu) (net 6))
 (segment (start 135.89 90.678) (end 135.382 91.186) (width 0.25) (layer F.Cu) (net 6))
 (segment (start 134.354 98.298) (end 134.366 98.286) (width 0.25) (layer F.Cu) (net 6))
 (segment (start 132.854 88.646) (end 132.854 87.872) (width 0.25) (layer F.Cu) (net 7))
 (segment (start 135.433 87.63) (end 137.481 89.678) (width 0.25) (layer F.Cu) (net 7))
 (segment (start 133.096 87.63) (end 135.433 87.63) (width 0.25) (layer F.Cu) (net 7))
 (segment (start 132.854 87.872) (end 133.096 87.63) (width 0.25) (layer F.Cu) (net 7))
 (segment (start 134.354 88.646) (end 134.354 96.774) (width 0.25) (layer F.Cu) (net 8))
 (segment (start 134.354 96.774) (end 134.366 96.786) (width 0.25) (layer F.Cu) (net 8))
 (segment (start 136.93902 83.82) (end 136.93902 79.77702) (width 0.25) (layer F.Cu) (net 9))
 (segment (start 136.93902 79.77702) (end 136.918 79.756) (width 0.25) (layer F.Cu) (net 9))
 (segment (start 141.974 79.756) (end 141.974 84.02898) (width 0.25) (layer F.Cu) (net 10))
 (segment (start 141.974 84.02898) (end 142.01902 84.074) (width 0.25) (layer F.Cu) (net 10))
 (segment (start 139.946 88.713) (end 139.946 84.09902) (width 0.25) (layer F.Cu) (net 11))
 (segment (start 139.946 84.09902) (end 139.92098 84.074) (width 0.25) (layer F.Cu) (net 11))
 (segment (start 142.52702 94.742) (end 145.034 94.742) (width 0.25) (layer F.Cu) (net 12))
 (segment (start 146.304 77.724) (end 144.514 77.724) (width 0.25) (layer F.Cu) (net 12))
 (via (at 146.304 77.724) (size 0.6) (drill 0.4) (layers F.Cu B.Cu) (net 12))
 (segment (start 146.304 93.472) (end 146.304 77.724) (width 0.25) (layer B.Cu) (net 12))
 (segment (start 145.034 94.742) (end 146.304 93.472) (width 0.25) (layer B.Cu) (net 12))
 (via (at 145.034 94.742) (size 0.6) (drill 0.4) (layers F.Cu B.Cu) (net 12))
 (segment (start 140.42898 94.742) (end 140.42898 92.66002) (width 0.25) (layer F.Cu) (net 13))
 (segment (start 140.42898 92.66002) (end 140.446 92.643) (width 0.25) (layer F.Cu) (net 13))
 (segment (start 148.844 97.79) (end 150.368 97.79) (width 0.25) (layer F.Cu) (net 14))
 (segment (start 155.956 92.202) (end 155.956 90.424) (width 0.25) (layer B.Cu) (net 14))
 (via (at 155.956 92.202) (size 0.6) (drill 0.4) (layers F.Cu B.Cu) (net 14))
 (segment (start 150.368 97.79) (end 155.956 92.202) (width 0.25) (layer F.Cu) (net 14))
 (segment (start 155.956 90.424) (end 156.21 90.424) (width 0.25) (layer B.Cu) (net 14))
 (segment (start 156.21 90.424) (end 158.242 88.392) (width 0.25) (layer B.Cu) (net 14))
 (segment (start 158.242 79.248) (end 156.718 77.724) (width 0.25) (layer F.Cu) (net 14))
 (via (at 158.242 79.248) (size 0.6) (drill 0.4) (layers F.Cu B.Cu) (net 14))
 (segment (start 158.242 88.392) (end 158.242 79.248) (width 0.25) (layer B.Cu) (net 14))
 (segment (start 156.718 77.724) (end 155.956 77.724) (width 0.25) (layer F.Cu) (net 14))
 (segment (start 155.702 90.424) (end 155.956 90.424) (width 0.25) (layer B.Cu) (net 14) (status 30))
 (segment (start 155.956 90.424) (end 156.972 90.424) (width 0.25) (layer B.Cu) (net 14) (status 30))
 (segment (start 138.446 88.713) (end 138.243 88.713) (width 0.25) (layer F.Cu) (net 20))
 (segment (start 153.924 80.264) (end 155.956 80.264) (width 0.25) (layer B.Cu) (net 20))
 (via (at 153.924 80.264) (size 0.6) (drill 0.4) (layers F.Cu B.Cu) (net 20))
 (segment (start 151.892 82.296) (end 153.924 80.264) (width 0.25) (layer F.Cu) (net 20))
 (via (at 151.892 82.296) (size 0.6) (drill 0.4) (layers F.Cu B.Cu) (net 20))
 (segment (start 150.622 82.296) (end 151.892 82.296) (width 0.25) (layer B.Cu) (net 20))
 (segment (start 148.59 84.328) (end 150.622 82.296) (width 0.25) (layer B.Cu) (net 20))
 (via (at 148.59 84.328) (size 0.6) (drill 0.4) (layers F.Cu B.Cu) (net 20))
 (segment (start 146.05 84.328) (end 148.59 84.328) (width 0.25) (layer F.Cu) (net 20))
 (segment (start 144.018 86.36) (end 146.05 84.328) (width 0.25) (layer F.Cu) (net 20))
 (via (at 144.018 86.36) (size 0.6) (drill 0.4) (layers F.Cu B.Cu) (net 20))
 (segment (start 142.748 87.63) (end 144.018 86.36) (width 0.25) (layer B.Cu) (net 20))
 (segment (start 137.16 87.63) (end 142.748 87.63) (width 0.25) (layer B.Cu) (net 20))
 (segment (start 136.906 87.376) (end 137.16 87.63) (width 0.25) (layer B.Cu) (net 20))
 (via (at 136.906 87.376) (size 0.6) (drill 0.4) (layers F.Cu B.Cu) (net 20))
 (segment (start 138.243 88.713) (end 136.906 87.376) (width 0.25) (layer F.Cu) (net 20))
 (segment (start 138.446 88.713) (end 138.446 88.662) (width 0.25) (layer F.Cu) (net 20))
 (segment (start 137.481 91.178) (end 136.406 91.178) (width 0.25) (layer F.Cu) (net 21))
 (segment (start 154.432 82.804) (end 155.956 82.804) (width 0.25) (layer B.Cu) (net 21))
 (segment (start 148.59 76.962) (end 154.432 82.804) (width 0.25) (layer B.Cu) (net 21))
 (segment (start 136.144 76.962) (end 148.59 76.962) (width 0.25) (layer B.Cu) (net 21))
 (segment (start 136.144 91.44) (end 136.144 76.962) (width 0.25) (layer B.Cu) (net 21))
 (via (at 136.144 91.44) (size 0.6) (drill 0.4) (layers F.Cu B.Cu) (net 21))
 (segment (start 136.406 91.178) (end 136.144 91.44) (width 0.25) (layer F.Cu) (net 21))
 (segment (start 149.848 82.55) (end 149.848 84.062) (width 0.25) (layer F.Cu) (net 22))
 (segment (start 153.67 87.884) (end 155.956 87.884) (width 0.25) (layer B.Cu) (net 22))
 (via (at 153.67 87.884) (size 0.6) (drill 0.4) (layers F.Cu B.Cu) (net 22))
 (segment (start 149.848 84.062) (end 153.67 87.884) (width 0.25) (layer F.Cu) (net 22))
 (segment (start 123.06808 79.89316) (end 123.06808 85.39226) (width 0.25) (layer B.Cu) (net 24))
 (segment (start 114.16792 79.89316) (end 123.06808 79.89316) (width 0.25) (layer B.Cu) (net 24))
 (segment (start 114.16792 85.39226) (end 114.16792 79.89316) (width 0.25) (layer B.Cu) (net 24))
 (segment (start 125.972 91.186) (end 125.972 95.492) (width 0.25) (layer F.Cu) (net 25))
 (segment (start 143.784222 91.240096) (end 141.411 91.178) (width 0.25) (layer F.Cu) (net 25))
 (segment (start 143.792222 91.248096) (end 143.784222 91.240096) (width 0.25) (layer F.Cu) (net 25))
 (via (at 143.792222 91.248096) (size 0.6) (drill 0.4) (layers F.Cu B.Cu) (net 25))
 (segment (start 143.764 96.774) (end 143.792222 91.248096) (width 0.25) (layer B.Cu) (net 25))
 (segment (start 142.748 96.774) (end 143.764 96.774) (width 0.25) (layer B.Cu) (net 25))
 (segment (start 127.254 96.774) (end 142.748 96.774) (width 0.25) (layer B.Cu) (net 25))
 (via (at 127.254 96.774) (size 0.6) (drill 0.4) (layers F.Cu B.Cu) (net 25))
 (segment (start 125.972 95.492) (end 127.254 96.774) (width 0.25) (layer F.Cu) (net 25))
 (segment (start 141.411 91.678) (end 142.994435 91.678) (width 0.25) (layer F.Cu) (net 26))
 (segment (start 130.556 93.98) (end 129.528 93.98) (width 0.25) (layer F.Cu) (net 26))
 (segment (start 132.588 96.012) (end 130.556 93.98) (width 0.25) (layer F.Cu) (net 26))
 (via (at 132.588 96.012) (size 0.6) (drill 0.4) (layers F.Cu B.Cu) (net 26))
 (segment (start 143.002 96.012) (end 132.588 96.012) (width 0.25) (layer B.Cu) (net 26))
 (segment (start 143.002 93.218) (end 143.002 96.012) (width 0.25) (layer B.Cu) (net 26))
 (via (at 143.002 93.218) (size 0.6) (drill 0.4) (layers F.Cu B.Cu) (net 26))
 (segment (start 143.002 91.685565) (end 143.002 93.218) (width 0.25) (layer F.Cu) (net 26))
 (segment (start 142.994435 91.678) (end 143.002 91.685565) (width 0.25) (layer F.Cu) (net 26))
 (segment (start 146.062 79.756) (end 145.288 79.756) (width 0.25) (layer F.Cu) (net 27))
 (segment (start 138.946 87.892) (end 138.946 88.713) (width 0.25) (layer F.Cu) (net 27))
 (segment (start 137.922 86.868) (end 138.946 87.892) (width 0.25) (layer F.Cu) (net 27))
 (via (at 137.922 86.868) (size 0.6) (drill 0.4) (layers F.Cu B.Cu) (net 27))
 (segment (start 137.922 82.296) (end 137.922 86.614) (width 0.25) (layer B.Cu) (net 27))
 (segment (start 137.922 82.296) (end 137.922 82.296) (width 0.25) (layer B.Cu) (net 27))
 (segment (start 142.748 82.296) (end 137.922 82.296) (width 0.25) (layer B.Cu) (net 27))
 (segment (start 143.002 82.042) (end 142.748 82.296) (width 0.25) (layer B.Cu) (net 27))
 (via (at 143.002 82.042) (size 0.6) (drill 0.4) (layers F.Cu B.Cu) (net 27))
 (segment (start 145.288 79.756) (end 143.002 82.042) (width 0.25) (layer F.Cu) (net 27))
 (segment (start 139.446 88.713) (end 139.446 87.122) (width 0.25) (layer F.Cu) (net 28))
 (segment (start 144.272 82.55) (end 148.348 82.55) (width 0.25) (layer F.Cu) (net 28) (status 20))
 (segment (start 144.018 82.804) (end 144.272 82.55) (width 0.25) (layer F.Cu) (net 28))
 (via (at 144.018 82.804) (size 0.6) (drill 0.4) (layers F.Cu B.Cu) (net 28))
 (segment (start 144.018 84.836) (end 144.018 82.804) (width 0.25) (layer B.Cu) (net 28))
 (segment (start 142.24 86.614) (end 144.018 84.836) (width 0.25) (layer B.Cu) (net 28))
 (segment (start 139.446 86.614) (end 142.24 86.614) (width 0.25) (layer B.Cu) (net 28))
 (segment (start 139.192 86.868) (end 139.446 86.614) (width 0.25) (layer B.Cu) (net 28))
 (via (at 139.192 86.868) (size 0.6) (drill 0.4) (layers F.Cu B.Cu) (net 28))
 (segment (start 139.446 87.122) (end 139.192 86.868) (width 0.25) (layer F.Cu) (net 28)))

